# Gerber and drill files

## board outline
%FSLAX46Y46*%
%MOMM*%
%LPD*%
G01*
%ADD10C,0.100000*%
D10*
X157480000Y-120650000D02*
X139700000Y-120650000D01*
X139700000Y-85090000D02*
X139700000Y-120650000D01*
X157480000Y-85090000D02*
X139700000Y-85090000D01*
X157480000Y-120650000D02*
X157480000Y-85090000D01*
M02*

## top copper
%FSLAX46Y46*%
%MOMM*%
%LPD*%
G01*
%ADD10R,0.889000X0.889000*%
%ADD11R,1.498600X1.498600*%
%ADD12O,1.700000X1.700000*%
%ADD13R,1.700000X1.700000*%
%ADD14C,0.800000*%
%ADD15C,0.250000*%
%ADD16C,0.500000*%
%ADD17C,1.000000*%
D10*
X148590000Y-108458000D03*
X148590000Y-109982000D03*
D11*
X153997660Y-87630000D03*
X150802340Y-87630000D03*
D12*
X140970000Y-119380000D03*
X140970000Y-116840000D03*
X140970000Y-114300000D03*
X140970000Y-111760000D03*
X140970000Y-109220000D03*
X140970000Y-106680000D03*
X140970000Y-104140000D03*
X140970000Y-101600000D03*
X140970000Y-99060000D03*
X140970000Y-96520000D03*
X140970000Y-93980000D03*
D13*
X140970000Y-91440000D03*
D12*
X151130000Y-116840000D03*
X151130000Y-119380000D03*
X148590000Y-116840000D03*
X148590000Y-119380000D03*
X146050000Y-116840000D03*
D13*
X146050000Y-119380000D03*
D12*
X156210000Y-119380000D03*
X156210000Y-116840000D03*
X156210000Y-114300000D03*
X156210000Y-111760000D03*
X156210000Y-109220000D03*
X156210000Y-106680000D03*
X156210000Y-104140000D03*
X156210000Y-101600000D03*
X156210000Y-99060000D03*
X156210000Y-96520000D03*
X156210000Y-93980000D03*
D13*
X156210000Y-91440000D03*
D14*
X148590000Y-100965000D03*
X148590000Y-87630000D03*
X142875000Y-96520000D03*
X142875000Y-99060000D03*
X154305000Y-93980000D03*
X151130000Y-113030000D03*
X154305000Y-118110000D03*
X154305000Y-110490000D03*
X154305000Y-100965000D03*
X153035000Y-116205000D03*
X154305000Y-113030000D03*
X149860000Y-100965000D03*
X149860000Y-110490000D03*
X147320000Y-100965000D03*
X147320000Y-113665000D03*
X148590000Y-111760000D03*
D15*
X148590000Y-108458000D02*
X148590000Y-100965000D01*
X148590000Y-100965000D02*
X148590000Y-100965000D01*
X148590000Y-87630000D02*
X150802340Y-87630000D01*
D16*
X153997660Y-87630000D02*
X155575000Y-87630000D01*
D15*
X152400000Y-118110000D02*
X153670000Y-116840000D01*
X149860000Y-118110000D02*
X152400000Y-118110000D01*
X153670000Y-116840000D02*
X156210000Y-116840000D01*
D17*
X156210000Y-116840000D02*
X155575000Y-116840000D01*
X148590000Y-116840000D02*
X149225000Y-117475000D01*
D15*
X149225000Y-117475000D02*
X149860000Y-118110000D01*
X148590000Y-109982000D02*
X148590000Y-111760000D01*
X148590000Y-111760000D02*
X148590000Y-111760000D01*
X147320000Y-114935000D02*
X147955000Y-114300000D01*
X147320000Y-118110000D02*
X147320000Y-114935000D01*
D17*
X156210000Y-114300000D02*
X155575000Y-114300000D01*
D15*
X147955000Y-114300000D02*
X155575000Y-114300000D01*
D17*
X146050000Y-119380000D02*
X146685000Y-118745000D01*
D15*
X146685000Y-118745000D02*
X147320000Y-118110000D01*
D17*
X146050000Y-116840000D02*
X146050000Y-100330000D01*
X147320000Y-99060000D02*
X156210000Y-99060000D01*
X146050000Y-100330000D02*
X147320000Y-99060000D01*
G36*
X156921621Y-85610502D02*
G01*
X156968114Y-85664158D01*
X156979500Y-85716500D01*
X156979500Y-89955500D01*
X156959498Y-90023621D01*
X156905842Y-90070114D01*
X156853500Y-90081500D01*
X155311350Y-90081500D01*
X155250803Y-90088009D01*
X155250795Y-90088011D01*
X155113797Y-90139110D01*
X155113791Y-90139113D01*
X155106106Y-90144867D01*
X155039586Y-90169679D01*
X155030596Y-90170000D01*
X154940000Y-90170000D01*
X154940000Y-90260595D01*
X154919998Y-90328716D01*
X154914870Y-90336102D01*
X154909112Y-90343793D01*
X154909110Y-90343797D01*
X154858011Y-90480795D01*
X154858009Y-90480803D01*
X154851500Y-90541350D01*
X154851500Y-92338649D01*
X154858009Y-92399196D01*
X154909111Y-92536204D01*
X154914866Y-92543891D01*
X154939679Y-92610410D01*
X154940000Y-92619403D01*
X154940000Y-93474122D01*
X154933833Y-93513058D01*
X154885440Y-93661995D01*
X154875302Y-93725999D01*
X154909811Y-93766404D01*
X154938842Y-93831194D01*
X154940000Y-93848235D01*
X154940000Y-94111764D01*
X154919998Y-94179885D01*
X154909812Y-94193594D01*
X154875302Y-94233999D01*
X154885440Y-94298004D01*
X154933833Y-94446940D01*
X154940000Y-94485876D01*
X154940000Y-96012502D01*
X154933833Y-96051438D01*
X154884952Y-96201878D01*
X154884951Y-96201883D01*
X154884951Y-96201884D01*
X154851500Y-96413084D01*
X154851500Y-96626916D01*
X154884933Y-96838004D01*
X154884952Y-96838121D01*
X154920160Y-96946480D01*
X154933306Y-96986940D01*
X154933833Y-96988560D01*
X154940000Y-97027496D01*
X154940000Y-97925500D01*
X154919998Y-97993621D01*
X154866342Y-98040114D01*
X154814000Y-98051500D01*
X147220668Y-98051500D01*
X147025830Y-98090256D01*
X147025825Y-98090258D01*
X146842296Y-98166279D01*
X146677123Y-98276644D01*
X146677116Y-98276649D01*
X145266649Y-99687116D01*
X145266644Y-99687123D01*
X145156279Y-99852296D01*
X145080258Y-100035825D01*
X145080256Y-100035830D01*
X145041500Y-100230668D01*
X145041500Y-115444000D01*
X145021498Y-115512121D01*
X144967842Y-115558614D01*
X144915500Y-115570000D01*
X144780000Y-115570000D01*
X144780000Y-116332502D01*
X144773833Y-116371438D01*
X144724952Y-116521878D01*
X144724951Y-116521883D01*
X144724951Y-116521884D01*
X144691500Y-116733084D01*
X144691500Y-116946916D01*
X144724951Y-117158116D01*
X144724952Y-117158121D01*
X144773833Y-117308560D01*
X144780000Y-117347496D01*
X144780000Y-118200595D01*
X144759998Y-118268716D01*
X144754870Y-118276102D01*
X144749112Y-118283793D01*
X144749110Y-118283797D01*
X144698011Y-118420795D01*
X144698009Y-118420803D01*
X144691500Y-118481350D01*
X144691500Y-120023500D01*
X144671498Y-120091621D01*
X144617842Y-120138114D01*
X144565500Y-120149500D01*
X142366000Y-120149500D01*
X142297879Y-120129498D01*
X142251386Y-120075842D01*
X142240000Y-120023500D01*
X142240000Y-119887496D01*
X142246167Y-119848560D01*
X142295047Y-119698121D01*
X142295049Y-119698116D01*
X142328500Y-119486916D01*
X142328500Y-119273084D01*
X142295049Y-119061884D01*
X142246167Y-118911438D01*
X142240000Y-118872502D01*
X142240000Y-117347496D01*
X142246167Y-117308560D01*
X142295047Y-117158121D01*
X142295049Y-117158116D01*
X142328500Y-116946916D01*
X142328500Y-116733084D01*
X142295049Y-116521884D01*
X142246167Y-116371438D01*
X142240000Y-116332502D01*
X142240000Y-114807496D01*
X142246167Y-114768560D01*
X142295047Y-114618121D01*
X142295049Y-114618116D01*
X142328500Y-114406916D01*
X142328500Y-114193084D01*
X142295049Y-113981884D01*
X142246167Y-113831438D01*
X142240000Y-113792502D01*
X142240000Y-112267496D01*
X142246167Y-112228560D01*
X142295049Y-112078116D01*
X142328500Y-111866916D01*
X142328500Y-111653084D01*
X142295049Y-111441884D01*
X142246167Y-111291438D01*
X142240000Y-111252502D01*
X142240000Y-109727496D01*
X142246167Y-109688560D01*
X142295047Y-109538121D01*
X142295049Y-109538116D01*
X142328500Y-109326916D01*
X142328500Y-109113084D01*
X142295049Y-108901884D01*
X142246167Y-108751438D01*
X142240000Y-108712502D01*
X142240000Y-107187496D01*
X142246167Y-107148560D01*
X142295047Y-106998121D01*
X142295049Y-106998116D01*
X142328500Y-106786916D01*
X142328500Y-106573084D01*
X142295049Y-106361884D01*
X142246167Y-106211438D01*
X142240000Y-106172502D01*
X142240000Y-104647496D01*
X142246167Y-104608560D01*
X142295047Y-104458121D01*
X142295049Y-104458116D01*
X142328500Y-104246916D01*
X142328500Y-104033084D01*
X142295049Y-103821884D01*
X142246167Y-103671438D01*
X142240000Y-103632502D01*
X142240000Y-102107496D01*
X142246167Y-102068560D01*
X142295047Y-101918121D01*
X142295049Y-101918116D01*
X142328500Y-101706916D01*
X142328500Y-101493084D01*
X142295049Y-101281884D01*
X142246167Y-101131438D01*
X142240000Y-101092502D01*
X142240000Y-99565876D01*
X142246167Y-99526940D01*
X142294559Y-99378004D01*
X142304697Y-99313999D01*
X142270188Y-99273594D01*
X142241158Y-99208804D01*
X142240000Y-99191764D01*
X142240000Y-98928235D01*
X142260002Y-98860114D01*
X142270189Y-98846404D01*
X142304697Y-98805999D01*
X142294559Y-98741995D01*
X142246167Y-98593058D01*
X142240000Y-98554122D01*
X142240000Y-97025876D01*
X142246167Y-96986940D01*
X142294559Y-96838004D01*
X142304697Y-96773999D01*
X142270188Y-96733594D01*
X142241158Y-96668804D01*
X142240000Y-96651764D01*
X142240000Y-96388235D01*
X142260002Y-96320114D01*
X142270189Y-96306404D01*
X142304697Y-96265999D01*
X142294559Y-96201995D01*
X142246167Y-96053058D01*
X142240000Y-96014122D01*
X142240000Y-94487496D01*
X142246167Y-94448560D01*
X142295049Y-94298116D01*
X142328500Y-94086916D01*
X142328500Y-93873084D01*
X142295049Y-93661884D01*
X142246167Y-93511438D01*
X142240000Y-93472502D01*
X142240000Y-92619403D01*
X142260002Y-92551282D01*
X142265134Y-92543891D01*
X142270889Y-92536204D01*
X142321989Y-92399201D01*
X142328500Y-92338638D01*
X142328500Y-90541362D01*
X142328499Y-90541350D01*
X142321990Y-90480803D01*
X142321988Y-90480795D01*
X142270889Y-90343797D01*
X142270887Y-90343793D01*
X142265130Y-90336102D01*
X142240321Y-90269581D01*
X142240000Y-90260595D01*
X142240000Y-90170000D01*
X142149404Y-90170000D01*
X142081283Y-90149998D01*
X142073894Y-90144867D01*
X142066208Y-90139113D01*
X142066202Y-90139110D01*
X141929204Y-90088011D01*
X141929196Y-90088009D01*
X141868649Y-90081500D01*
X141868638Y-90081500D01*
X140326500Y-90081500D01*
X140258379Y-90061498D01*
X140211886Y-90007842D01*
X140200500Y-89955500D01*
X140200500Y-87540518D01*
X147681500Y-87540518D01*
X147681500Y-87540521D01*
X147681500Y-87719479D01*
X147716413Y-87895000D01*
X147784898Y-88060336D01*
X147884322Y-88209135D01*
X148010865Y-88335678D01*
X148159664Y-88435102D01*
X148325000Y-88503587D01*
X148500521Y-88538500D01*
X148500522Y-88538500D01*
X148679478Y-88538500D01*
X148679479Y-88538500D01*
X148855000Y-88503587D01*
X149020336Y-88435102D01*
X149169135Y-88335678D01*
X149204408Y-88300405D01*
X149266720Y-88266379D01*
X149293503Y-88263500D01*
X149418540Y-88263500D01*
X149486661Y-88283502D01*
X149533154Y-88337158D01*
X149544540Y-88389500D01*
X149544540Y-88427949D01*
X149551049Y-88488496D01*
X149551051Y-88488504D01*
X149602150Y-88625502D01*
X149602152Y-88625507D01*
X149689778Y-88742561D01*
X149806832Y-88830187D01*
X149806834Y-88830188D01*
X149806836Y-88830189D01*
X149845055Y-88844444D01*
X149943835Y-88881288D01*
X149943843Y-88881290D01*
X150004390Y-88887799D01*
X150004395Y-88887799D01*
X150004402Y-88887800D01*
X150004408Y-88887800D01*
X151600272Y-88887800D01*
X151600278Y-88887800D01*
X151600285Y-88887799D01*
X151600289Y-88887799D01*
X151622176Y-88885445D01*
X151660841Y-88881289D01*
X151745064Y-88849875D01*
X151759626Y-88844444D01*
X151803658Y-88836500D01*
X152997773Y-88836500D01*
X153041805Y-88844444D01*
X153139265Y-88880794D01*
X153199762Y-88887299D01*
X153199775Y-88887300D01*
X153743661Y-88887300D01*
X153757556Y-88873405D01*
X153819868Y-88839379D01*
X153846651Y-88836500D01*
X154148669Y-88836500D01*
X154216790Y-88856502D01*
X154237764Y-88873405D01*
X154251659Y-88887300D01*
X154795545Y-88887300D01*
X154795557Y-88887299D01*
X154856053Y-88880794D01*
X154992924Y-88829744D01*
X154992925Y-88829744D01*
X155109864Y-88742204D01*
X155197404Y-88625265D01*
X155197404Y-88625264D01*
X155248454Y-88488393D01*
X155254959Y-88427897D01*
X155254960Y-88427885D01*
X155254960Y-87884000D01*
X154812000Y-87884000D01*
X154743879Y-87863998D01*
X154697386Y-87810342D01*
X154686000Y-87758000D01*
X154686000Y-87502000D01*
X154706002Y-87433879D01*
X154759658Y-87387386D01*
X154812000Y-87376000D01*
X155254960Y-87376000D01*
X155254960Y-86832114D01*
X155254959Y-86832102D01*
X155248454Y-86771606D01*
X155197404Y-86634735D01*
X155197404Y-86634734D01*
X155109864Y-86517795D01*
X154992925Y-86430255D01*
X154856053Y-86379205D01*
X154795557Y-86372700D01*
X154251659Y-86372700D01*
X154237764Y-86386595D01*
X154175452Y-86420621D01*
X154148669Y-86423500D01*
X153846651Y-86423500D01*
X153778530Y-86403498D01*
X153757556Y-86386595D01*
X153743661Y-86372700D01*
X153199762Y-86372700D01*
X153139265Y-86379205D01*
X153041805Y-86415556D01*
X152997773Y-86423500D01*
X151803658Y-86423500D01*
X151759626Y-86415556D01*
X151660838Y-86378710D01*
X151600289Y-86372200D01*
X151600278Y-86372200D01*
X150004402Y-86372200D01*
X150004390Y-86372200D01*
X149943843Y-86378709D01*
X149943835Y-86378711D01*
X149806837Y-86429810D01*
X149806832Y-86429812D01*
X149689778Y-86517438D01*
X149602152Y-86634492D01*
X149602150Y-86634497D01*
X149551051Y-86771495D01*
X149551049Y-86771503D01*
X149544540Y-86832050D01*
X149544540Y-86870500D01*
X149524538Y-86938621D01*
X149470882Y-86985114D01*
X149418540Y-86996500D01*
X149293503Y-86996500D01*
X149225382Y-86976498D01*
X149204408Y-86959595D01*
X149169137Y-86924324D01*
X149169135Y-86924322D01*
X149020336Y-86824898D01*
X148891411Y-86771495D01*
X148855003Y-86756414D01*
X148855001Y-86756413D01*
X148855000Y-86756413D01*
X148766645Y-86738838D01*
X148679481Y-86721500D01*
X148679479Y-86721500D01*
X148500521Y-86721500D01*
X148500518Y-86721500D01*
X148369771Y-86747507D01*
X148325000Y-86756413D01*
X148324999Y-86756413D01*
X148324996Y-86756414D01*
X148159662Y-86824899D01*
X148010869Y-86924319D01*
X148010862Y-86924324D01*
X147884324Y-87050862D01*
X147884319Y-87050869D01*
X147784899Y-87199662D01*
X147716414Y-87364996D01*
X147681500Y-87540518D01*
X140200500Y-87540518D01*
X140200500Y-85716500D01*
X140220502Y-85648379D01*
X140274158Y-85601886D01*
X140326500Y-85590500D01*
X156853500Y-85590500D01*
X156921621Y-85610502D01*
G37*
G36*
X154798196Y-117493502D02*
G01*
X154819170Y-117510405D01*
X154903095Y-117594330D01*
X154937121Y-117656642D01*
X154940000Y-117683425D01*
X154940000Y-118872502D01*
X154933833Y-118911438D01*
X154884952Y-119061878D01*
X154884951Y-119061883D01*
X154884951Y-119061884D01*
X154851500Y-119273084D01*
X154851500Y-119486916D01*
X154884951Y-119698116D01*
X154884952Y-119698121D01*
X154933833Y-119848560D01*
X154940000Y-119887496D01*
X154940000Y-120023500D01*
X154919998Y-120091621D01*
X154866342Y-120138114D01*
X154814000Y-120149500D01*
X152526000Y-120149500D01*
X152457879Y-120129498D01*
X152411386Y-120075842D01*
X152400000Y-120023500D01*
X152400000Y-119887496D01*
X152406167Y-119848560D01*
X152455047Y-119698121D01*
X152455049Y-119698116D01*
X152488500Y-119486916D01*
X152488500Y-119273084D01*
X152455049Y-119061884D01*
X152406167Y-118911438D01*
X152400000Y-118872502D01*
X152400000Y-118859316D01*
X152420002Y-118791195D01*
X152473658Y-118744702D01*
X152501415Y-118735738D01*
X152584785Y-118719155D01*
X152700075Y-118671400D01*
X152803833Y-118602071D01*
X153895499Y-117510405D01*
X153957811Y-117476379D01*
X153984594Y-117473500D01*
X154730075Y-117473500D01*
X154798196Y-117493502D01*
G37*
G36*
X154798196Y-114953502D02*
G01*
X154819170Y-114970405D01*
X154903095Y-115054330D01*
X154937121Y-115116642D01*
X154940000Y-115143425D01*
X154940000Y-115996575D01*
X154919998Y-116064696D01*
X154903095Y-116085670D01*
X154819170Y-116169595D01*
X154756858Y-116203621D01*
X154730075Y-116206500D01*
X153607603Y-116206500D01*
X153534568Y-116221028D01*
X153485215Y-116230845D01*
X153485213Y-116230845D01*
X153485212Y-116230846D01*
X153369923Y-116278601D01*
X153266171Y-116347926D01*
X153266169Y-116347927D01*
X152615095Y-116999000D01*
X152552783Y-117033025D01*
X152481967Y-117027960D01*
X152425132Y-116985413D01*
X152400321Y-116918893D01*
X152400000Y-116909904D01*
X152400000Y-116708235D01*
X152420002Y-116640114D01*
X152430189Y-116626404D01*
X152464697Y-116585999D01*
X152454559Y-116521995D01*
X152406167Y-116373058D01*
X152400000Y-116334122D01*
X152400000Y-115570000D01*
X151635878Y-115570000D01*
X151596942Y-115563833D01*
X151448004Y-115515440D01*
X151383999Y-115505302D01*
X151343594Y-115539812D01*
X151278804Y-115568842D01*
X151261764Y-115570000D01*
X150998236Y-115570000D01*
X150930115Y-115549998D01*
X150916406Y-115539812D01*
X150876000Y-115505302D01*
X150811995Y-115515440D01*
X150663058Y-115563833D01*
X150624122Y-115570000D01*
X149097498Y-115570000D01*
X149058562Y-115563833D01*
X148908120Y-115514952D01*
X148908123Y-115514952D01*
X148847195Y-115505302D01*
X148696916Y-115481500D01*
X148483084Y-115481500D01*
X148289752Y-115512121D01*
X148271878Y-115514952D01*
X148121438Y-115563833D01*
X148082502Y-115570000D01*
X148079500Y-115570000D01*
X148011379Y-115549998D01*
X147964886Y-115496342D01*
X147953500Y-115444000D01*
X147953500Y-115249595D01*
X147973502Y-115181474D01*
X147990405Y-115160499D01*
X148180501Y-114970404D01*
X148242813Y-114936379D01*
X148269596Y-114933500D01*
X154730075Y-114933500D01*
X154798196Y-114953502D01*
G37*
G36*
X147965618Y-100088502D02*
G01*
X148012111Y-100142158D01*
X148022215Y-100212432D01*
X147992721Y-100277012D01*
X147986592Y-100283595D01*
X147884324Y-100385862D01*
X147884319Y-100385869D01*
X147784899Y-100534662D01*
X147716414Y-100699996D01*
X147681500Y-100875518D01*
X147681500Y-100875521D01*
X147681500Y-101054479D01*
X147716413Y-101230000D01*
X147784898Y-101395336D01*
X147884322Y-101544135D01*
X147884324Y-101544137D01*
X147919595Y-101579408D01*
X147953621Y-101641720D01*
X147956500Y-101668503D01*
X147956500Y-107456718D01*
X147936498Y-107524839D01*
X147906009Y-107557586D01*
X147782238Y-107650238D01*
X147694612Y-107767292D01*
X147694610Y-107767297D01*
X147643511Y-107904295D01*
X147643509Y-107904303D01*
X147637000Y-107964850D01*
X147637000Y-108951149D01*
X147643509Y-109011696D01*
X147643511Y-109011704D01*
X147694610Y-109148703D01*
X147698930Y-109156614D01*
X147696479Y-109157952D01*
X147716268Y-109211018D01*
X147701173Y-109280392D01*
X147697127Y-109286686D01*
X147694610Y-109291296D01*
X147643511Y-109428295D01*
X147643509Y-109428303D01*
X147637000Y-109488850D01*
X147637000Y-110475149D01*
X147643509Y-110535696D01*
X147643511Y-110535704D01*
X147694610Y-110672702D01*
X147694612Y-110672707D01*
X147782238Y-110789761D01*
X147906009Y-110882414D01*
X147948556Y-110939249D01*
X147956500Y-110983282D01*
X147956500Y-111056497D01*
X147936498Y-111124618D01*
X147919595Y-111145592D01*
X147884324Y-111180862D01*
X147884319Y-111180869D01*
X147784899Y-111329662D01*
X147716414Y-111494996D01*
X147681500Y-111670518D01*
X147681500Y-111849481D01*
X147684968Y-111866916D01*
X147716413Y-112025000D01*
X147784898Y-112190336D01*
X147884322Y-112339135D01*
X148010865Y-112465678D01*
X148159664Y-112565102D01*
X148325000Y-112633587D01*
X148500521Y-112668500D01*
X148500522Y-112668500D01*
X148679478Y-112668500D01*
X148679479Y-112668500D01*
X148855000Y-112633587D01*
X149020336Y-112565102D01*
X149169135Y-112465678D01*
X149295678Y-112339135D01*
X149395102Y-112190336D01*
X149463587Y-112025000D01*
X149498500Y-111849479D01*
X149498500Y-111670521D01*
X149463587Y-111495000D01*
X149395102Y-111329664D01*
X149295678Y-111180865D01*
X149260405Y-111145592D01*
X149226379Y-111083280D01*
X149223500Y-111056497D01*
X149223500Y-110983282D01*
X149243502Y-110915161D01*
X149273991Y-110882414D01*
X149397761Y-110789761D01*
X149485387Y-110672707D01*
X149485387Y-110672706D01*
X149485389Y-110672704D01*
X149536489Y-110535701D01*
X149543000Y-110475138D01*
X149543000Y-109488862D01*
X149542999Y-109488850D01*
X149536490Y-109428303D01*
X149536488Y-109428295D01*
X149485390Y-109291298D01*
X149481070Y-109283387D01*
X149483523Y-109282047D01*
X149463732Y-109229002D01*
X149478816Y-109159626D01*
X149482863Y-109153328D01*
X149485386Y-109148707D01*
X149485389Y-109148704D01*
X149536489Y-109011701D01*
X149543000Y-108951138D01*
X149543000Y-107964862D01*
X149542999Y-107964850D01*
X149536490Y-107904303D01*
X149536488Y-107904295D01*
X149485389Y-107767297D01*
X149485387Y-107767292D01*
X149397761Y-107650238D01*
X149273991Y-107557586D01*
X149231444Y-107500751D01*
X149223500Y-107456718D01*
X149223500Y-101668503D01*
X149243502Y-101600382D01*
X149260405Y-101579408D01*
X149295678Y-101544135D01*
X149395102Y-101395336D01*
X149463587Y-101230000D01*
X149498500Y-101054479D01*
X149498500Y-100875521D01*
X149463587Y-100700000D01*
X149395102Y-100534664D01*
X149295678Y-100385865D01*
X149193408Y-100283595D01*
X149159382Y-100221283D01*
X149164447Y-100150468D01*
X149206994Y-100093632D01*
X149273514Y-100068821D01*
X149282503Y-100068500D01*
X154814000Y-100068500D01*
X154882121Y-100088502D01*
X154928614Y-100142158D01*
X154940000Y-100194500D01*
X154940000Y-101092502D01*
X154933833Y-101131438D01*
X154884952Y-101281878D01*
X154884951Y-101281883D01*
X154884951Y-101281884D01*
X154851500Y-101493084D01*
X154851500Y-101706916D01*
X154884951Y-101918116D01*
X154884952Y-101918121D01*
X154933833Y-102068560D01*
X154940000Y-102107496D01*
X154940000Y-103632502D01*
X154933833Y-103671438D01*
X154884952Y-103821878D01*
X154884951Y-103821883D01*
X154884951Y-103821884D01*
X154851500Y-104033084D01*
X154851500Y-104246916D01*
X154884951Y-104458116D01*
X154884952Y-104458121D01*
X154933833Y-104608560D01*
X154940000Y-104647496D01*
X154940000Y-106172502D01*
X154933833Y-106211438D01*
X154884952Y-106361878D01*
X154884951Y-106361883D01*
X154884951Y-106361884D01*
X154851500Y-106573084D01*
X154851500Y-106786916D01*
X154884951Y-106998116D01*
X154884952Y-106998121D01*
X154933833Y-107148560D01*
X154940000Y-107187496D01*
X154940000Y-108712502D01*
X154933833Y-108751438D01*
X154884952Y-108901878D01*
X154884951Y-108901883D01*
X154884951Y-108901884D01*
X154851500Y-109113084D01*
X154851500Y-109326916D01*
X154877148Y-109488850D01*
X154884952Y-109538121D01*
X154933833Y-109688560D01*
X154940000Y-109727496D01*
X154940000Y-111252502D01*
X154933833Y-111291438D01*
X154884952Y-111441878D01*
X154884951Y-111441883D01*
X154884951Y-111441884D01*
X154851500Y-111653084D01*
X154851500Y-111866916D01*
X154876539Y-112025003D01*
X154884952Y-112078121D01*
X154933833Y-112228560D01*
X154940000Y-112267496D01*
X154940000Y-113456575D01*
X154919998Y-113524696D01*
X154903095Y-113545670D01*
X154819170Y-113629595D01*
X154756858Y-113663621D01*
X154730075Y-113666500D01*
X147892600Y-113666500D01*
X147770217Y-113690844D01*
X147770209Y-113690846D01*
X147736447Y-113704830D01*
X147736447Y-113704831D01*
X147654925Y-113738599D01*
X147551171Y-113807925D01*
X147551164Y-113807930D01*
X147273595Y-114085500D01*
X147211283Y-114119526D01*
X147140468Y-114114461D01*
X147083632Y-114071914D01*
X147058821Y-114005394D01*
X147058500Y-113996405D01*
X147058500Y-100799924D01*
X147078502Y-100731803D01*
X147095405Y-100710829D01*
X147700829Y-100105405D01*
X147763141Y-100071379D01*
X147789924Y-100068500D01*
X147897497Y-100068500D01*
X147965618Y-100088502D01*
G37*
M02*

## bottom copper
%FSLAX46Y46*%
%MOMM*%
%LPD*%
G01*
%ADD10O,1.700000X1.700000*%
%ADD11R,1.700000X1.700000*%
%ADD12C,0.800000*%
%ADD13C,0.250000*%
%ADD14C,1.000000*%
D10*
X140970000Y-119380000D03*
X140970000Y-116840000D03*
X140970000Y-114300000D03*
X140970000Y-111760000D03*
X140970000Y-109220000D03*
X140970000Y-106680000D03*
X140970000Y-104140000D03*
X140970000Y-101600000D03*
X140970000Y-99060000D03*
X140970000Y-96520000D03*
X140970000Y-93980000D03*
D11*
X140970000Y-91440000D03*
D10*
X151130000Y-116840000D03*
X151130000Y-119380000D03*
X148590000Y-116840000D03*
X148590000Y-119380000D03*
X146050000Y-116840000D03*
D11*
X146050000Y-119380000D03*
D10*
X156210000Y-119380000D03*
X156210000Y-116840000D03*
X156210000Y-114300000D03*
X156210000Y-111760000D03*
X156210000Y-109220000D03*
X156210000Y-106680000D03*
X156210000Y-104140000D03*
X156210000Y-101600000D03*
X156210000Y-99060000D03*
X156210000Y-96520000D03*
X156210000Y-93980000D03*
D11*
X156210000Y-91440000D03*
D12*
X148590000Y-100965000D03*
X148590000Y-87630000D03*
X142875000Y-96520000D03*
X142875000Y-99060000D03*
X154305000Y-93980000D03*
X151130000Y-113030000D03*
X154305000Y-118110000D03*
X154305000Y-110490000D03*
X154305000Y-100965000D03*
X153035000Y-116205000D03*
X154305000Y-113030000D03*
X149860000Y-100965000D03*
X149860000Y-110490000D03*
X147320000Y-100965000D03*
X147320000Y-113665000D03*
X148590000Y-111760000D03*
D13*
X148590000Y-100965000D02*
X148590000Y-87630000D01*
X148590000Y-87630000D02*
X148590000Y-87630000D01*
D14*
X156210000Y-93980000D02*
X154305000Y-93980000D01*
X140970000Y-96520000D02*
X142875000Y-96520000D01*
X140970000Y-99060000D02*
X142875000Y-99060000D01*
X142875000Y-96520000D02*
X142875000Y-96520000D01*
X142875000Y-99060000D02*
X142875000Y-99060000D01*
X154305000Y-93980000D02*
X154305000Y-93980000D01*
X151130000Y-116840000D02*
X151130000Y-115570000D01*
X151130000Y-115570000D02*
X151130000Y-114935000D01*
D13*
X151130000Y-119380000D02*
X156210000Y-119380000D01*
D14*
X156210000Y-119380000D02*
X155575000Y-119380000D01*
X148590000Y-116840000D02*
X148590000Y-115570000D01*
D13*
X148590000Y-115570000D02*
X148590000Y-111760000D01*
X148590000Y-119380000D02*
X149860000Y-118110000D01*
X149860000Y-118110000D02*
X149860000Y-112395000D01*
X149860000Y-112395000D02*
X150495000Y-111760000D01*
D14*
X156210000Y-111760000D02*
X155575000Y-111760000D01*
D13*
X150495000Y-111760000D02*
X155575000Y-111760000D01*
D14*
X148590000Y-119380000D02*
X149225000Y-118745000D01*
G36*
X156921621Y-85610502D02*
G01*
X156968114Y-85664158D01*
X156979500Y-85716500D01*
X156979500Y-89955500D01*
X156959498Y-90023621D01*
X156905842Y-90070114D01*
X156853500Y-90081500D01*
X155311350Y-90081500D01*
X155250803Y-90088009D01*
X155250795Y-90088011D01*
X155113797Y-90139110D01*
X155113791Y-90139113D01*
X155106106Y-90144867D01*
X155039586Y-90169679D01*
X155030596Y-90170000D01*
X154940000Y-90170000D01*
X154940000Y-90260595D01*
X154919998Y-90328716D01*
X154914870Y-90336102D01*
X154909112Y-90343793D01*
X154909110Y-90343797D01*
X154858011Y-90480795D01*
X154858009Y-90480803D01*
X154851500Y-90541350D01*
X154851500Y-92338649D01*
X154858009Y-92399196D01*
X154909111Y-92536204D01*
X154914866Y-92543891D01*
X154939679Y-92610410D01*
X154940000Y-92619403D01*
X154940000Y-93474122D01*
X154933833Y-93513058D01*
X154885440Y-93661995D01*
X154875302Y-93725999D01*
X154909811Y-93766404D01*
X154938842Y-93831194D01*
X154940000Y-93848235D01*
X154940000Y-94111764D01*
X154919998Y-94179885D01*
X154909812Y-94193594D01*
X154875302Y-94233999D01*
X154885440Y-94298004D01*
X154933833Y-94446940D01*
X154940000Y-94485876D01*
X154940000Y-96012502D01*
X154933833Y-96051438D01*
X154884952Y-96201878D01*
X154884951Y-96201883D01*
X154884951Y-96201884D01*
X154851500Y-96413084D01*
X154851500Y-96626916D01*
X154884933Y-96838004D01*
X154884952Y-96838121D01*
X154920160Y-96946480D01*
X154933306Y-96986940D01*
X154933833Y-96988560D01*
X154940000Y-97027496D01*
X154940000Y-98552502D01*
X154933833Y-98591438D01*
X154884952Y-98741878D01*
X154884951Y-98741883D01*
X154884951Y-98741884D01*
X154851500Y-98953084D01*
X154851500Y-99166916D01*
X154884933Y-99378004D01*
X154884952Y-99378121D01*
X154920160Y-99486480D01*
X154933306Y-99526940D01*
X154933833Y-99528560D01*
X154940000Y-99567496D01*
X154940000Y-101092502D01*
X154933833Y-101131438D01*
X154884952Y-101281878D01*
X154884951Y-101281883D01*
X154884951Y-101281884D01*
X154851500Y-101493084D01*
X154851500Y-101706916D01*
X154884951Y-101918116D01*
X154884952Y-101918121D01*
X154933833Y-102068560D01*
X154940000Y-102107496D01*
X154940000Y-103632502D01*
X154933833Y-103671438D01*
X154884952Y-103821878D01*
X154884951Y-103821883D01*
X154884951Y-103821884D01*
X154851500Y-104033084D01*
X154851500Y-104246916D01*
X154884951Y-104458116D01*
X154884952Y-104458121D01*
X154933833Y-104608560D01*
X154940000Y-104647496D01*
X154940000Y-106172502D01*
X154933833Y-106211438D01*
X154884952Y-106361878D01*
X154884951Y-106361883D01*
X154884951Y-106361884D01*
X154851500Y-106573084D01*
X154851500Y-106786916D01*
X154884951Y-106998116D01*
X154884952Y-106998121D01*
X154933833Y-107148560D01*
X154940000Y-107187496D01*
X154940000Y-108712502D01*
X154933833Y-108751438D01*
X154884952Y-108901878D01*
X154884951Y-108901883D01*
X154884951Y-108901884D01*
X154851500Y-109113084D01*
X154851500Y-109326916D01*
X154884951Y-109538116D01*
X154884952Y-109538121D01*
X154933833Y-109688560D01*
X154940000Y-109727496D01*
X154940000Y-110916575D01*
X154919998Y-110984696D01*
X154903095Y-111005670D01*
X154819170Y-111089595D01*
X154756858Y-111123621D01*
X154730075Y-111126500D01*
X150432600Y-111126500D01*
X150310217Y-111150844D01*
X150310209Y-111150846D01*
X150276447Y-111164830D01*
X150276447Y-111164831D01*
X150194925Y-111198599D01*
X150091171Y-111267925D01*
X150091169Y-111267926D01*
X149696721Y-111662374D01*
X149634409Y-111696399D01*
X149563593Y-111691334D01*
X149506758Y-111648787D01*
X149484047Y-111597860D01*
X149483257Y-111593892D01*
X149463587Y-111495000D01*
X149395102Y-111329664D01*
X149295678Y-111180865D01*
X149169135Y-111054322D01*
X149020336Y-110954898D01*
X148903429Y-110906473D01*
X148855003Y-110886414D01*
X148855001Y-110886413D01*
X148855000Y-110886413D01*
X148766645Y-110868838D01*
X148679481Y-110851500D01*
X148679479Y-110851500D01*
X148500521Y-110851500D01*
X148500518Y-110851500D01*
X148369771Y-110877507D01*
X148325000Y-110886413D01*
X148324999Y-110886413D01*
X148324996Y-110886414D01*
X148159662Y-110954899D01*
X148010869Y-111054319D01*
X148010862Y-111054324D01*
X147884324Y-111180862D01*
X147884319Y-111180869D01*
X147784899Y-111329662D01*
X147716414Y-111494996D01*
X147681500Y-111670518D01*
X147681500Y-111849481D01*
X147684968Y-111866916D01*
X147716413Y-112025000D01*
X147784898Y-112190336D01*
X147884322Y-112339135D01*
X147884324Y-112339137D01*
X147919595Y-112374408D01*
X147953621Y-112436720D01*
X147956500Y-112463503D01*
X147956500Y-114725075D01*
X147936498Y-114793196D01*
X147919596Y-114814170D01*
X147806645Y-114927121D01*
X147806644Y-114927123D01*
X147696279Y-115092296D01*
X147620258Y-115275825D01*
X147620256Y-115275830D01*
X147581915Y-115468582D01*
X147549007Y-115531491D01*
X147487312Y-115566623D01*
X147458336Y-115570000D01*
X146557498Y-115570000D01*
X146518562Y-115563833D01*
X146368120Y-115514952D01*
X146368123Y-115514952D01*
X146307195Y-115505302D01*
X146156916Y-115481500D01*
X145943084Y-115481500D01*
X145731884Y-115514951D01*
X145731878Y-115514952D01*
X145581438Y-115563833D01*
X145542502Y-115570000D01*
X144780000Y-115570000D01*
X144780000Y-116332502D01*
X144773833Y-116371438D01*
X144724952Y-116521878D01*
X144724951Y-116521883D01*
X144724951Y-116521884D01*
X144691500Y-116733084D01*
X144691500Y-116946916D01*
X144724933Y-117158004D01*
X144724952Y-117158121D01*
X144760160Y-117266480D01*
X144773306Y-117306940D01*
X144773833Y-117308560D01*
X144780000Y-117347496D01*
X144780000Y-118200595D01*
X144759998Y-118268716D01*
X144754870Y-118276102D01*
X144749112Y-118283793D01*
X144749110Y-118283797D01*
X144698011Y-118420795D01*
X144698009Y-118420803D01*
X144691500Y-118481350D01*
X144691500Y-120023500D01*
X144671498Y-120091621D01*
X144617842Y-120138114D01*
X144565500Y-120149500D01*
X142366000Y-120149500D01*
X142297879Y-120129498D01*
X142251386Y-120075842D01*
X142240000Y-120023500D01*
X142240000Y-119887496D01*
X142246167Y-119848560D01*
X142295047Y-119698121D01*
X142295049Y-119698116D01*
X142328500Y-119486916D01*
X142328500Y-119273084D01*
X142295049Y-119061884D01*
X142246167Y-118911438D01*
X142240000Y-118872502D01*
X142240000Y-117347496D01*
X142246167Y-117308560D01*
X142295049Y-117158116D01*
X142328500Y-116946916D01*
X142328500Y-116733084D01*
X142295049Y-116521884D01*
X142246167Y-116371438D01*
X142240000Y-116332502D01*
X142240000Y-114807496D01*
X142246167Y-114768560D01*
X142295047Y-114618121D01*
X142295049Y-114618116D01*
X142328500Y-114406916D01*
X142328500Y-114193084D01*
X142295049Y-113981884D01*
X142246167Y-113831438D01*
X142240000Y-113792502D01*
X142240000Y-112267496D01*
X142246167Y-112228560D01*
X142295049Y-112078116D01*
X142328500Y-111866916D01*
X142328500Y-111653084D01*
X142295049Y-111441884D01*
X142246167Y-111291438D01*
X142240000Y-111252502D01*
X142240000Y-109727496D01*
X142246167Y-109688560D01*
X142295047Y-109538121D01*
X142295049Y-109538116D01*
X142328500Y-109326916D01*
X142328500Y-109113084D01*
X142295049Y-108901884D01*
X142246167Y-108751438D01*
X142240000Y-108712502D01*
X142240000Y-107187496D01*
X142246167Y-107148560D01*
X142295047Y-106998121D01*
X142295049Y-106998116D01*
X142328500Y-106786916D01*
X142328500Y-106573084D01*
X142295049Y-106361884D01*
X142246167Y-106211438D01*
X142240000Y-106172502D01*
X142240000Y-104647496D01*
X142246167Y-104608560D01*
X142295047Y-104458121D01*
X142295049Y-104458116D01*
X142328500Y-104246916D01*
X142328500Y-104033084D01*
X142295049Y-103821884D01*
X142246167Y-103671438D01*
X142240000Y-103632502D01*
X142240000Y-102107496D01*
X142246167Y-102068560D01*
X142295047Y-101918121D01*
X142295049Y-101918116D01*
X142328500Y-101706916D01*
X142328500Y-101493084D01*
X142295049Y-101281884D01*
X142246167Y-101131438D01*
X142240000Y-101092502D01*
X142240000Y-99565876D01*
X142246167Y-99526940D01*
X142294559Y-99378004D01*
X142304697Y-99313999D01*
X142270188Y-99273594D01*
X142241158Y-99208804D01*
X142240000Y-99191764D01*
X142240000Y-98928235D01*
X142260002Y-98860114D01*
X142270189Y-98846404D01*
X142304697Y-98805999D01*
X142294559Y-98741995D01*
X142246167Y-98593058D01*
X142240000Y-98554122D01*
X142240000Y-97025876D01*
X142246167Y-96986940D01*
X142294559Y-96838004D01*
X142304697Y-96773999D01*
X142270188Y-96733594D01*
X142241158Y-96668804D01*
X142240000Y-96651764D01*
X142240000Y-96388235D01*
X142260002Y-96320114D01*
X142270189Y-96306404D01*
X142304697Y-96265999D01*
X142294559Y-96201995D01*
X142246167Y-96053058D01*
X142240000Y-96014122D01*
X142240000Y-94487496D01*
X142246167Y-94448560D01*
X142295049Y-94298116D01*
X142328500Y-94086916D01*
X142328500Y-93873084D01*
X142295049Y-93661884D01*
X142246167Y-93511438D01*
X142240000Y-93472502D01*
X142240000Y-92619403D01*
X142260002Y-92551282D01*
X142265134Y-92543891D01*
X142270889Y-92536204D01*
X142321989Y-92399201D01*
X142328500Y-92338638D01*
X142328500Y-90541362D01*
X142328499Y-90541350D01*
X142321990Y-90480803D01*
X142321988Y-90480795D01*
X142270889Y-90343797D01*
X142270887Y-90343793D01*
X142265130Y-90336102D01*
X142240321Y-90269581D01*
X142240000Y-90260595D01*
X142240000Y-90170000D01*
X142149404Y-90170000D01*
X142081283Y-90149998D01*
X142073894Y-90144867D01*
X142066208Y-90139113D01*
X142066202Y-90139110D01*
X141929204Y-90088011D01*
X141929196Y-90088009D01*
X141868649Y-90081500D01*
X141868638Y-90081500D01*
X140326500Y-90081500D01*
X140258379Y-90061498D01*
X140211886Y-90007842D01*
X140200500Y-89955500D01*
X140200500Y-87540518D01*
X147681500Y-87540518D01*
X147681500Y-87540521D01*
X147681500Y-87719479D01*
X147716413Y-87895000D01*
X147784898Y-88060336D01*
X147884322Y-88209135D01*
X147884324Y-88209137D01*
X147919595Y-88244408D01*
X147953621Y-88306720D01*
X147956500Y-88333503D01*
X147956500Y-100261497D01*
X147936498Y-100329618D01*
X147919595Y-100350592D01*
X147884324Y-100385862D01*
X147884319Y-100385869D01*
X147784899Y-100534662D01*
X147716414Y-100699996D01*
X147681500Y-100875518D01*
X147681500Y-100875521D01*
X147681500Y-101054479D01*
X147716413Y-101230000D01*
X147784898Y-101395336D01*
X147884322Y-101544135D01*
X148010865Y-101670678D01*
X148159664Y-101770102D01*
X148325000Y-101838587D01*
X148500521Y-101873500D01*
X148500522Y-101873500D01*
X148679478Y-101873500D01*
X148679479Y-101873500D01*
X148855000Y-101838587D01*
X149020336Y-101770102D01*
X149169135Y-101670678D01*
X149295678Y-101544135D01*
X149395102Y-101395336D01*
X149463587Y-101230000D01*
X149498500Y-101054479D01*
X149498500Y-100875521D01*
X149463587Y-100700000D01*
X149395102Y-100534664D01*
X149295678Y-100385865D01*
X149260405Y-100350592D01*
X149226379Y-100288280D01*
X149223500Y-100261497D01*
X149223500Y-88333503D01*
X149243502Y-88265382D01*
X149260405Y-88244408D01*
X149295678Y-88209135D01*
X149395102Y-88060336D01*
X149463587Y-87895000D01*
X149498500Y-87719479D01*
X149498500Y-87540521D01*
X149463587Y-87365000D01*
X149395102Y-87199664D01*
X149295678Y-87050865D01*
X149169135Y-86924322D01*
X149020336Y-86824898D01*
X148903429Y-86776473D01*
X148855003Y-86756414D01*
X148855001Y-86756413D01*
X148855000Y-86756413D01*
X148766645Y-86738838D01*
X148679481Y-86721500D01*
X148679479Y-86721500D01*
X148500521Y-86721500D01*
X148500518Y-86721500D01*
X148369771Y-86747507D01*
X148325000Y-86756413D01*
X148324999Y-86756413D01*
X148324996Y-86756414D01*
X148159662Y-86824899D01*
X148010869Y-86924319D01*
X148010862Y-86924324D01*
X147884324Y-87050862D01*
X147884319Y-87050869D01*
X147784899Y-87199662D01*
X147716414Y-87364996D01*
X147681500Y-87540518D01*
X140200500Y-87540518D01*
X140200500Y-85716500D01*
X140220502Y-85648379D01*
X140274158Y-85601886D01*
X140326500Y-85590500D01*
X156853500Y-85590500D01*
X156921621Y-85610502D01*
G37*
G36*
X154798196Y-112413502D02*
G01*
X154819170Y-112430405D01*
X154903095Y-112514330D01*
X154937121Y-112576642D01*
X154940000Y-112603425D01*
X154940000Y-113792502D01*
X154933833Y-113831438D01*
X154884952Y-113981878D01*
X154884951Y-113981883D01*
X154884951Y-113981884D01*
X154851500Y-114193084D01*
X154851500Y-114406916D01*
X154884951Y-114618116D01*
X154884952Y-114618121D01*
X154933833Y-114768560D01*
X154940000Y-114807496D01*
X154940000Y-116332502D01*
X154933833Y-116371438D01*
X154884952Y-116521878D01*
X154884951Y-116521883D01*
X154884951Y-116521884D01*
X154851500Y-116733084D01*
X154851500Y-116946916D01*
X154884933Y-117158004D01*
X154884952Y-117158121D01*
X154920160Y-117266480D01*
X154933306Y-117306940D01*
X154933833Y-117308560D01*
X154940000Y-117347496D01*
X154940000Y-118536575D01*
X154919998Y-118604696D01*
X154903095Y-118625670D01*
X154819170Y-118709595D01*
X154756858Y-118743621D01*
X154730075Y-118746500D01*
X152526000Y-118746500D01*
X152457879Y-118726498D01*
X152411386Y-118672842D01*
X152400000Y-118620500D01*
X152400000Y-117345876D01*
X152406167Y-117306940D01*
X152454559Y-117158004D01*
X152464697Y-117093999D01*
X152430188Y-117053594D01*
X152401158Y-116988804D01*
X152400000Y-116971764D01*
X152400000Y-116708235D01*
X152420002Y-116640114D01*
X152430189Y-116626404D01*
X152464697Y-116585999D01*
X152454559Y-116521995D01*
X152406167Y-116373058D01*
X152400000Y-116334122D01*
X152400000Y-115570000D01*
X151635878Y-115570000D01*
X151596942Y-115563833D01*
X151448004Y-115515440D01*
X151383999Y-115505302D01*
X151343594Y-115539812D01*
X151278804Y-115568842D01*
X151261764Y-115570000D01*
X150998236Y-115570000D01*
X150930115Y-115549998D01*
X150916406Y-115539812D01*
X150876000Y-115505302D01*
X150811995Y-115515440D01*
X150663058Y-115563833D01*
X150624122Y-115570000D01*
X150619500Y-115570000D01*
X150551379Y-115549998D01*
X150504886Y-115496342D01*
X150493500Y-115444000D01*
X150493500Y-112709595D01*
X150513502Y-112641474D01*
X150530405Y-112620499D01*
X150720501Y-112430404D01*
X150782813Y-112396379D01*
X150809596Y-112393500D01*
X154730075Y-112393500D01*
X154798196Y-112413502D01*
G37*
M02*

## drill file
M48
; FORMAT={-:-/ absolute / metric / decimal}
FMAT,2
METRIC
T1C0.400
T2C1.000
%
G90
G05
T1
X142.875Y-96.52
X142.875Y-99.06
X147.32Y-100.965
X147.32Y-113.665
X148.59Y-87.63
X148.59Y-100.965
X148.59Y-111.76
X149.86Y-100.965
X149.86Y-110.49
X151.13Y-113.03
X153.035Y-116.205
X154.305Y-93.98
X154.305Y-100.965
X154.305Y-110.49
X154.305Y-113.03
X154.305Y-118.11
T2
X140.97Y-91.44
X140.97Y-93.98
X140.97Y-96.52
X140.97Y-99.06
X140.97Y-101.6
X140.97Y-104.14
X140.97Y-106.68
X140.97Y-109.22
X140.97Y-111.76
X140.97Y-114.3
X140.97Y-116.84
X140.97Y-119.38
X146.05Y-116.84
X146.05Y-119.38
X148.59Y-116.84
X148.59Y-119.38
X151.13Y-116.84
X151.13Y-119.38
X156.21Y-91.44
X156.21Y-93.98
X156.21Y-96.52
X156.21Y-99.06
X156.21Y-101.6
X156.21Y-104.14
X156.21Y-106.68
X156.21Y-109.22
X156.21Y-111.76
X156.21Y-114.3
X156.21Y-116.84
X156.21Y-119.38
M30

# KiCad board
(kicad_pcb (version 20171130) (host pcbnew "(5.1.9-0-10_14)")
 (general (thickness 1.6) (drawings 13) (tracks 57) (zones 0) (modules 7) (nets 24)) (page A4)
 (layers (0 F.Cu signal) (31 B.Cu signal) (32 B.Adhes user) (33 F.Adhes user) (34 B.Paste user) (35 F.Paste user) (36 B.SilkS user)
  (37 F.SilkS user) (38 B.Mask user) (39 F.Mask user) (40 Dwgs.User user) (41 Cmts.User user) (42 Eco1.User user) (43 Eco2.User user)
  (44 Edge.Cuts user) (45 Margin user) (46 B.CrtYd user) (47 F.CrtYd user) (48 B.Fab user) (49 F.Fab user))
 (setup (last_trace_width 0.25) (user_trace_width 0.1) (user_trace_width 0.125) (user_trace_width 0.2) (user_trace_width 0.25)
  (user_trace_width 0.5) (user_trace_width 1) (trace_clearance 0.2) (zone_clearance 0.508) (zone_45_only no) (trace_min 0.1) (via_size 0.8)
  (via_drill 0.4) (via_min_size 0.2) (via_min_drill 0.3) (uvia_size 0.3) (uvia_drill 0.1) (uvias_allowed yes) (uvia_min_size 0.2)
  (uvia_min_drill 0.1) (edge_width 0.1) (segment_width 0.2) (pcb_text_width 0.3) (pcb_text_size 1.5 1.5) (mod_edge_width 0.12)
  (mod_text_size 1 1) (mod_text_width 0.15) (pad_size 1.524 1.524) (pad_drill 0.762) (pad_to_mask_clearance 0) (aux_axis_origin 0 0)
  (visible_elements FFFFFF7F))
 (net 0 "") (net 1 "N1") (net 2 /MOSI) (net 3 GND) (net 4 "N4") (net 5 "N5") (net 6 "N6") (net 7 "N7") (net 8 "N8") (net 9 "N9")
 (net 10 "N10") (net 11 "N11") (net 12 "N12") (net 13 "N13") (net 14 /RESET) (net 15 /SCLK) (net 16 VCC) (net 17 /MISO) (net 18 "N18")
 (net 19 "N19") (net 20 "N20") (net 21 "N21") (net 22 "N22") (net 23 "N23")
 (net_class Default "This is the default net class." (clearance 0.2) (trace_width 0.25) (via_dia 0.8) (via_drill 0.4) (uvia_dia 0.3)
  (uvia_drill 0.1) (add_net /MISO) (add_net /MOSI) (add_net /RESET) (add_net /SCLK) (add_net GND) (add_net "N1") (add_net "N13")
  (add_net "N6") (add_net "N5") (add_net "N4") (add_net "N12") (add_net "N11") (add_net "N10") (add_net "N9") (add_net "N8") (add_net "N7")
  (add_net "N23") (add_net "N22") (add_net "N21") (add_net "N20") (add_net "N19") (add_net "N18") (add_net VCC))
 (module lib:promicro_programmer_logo (layer B.Cu) (at 146.05 93.98 270)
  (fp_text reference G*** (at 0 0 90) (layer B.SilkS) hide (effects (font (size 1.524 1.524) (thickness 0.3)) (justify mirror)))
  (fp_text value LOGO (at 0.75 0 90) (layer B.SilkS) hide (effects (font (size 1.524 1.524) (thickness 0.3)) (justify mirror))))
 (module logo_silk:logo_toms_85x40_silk (layer B.Cu) (at 146.685 106.68 270)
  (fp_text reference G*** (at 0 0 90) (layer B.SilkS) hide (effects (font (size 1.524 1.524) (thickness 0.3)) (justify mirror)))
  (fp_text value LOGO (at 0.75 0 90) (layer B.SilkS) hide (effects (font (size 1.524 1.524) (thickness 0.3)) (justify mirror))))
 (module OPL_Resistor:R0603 (layer F.Cu) (at 148.59 109.22 90)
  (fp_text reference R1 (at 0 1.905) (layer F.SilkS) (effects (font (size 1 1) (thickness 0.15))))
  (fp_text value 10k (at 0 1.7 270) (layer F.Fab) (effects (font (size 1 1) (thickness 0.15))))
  (pad 2 smd rect (at 0.762 0 90) (size 0.889 0.889) (layers F.Cu F.Paste F.Mask) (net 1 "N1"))
  (pad 1 smd rect (at -0.762 0 90) (size 0.889 0.889) (layers F.Cu F.Paste F.Mask) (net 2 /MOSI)))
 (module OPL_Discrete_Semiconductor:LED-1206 (layer F.Cu) (at 152.4 87.63 180)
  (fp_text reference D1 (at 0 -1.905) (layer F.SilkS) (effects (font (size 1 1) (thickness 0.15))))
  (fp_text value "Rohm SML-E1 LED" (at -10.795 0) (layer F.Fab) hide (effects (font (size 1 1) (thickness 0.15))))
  (pad 1 smd rect (at -1.59766 0 180) (size 1.4986 1.4986) (layers F.Cu F.Paste F.Mask) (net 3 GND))
  (pad 2 smd rect (at 1.59766 0 180) (size 1.4986 1.4986) (layers F.Cu F.Paste F.Mask) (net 1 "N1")))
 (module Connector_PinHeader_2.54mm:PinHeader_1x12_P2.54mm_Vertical (layer F.Cu) (at 140.97 91.44)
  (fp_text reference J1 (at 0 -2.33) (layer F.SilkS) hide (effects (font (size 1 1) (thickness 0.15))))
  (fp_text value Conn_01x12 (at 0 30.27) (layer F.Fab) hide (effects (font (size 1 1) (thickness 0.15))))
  (pad 12 thru_hole oval (at 0 27.94) (size 1.7 1.7) (drill 1) (layers *.Cu *.Mask) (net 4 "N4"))
  (pad 11 thru_hole oval (at 0 25.4) (size 1.7 1.7) (drill 1) (layers *.Cu *.Mask) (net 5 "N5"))
  (pad 10 thru_hole oval (at 0 22.86) (size 1.7 1.7) (drill 1) (layers *.Cu *.Mask) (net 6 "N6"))
  (pad 9 thru_hole oval (at 0 20.32) (size 1.7 1.7) (drill 1) (layers *.Cu *.Mask) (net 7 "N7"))
  (pad 8 thru_hole oval (at 0 17.78) (size 1.7 1.7) (drill 1) (layers *.Cu *.Mask) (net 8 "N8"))
  (pad 7 thru_hole oval (at 0 15.24) (size 1.7 1.7) (drill 1) (layers *.Cu *.Mask) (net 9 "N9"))
  (pad 6 thru_hole oval (at 0 12.7) (size 1.7 1.7) (drill 1) (layers *.Cu *.Mask) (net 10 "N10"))
  (pad 5 thru_hole oval (at 0 10.16) (size 1.7 1.7) (drill 1) (layers *.Cu *.Mask) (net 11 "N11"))
  (pad 4 thru_hole oval (at 0 7.62) (size 1.7 1.7) (drill 1) (layers *.Cu *.Mask) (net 3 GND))
  (pad 3 thru_hole oval (at 0 5.08) (size 1.7 1.7) (drill 1) (layers *.Cu *.Mask) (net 3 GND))
  (pad 2 thru_hole oval (at 0 2.54) (size 1.7 1.7) (drill 1) (layers *.Cu *.Mask) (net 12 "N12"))
  (pad 1 thru_hole rect (at 0 0) (size 1.7 1.7) (drill 1) (layers *.Cu *.Mask) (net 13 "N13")))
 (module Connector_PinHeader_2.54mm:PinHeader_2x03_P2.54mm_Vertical (layer F.Cu) (at 146.05 119.38 90)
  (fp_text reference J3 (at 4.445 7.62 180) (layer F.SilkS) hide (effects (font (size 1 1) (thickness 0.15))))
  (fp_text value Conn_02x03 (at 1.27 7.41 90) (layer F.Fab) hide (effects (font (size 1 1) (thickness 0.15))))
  (pad 6 thru_hole oval (at 2.54 5.08 90) (size 1.7 1.7) (drill 1) (layers *.Cu *.Mask) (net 3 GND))
  (pad 5 thru_hole oval (at 0 5.08 90) (size 1.7 1.7) (drill 1) (layers *.Cu *.Mask) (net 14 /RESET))
  (pad 4 thru_hole oval (at 2.54 2.54 90) (size 1.7 1.7) (drill 1) (layers *.Cu *.Mask) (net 2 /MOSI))
  (pad 3 thru_hole oval (at 0 2.54 90) (size 1.7 1.7) (drill 1) (layers *.Cu *.Mask) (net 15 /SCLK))
  (pad 2 thru_hole oval (at 2.54 0 90) (size 1.7 1.7) (drill 1) (layers *.Cu *.Mask) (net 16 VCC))
  (pad 1 thru_hole rect (at 0 0 90) (size 1.7 1.7) (drill 1) (layers *.Cu *.Mask) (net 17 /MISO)))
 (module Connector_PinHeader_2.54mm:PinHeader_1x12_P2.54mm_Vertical (layer F.Cu) (at 156.21 91.44)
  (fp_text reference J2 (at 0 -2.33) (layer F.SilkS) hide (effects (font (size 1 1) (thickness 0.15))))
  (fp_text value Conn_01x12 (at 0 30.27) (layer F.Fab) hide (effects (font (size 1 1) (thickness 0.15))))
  (pad 12 thru_hole oval (at 0 27.94) (size 1.7 1.7) (drill 1) (layers *.Cu *.Mask) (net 14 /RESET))
  (pad 11 thru_hole oval (at 0 25.4) (size 1.7 1.7) (drill 1) (layers *.Cu *.Mask) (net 2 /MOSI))
  (pad 10 thru_hole oval (at 0 22.86) (size 1.7 1.7) (drill 1) (layers *.Cu *.Mask) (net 17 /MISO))
  (pad 9 thru_hole oval (at 0 20.32) (size 1.7 1.7) (drill 1) (layers *.Cu *.Mask) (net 15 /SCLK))
  (pad 8 thru_hole oval (at 0 17.78) (size 1.7 1.7) (drill 1) (layers *.Cu *.Mask) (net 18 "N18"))
  (pad 7 thru_hole oval (at 0 15.24) (size 1.7 1.7) (drill 1) (layers *.Cu *.Mask) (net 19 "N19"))
  (pad 6 thru_hole oval (at 0 12.7) (size 1.7 1.7) (drill 1) (layers *.Cu *.Mask) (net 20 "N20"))
  (pad 5 thru_hole oval (at 0 10.16) (size 1.7 1.7) (drill 1) (layers *.Cu *.Mask) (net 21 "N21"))
  (pad 4 thru_hole oval (at 0 7.62) (size 1.7 1.7) (drill 1) (layers *.Cu *.Mask) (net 16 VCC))
  (pad 3 thru_hole oval (at 0 5.08) (size 1.7 1.7) (drill 1) (layers *.Cu *.Mask) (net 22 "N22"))
  (pad 2 thru_hole oval (at 0 2.54) (size 1.7 1.7) (drill 1) (layers *.Cu *.Mask) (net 3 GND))
  (pad 1 thru_hole rect (at 0 0) (size 1.7 1.7) (drill 1) (layers *.Cu *.Mask) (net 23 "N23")))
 (gr_line (start 157.48 120.65) (end 139.7 120.65) (layer Edge.Cuts) (width 0.1))
 (gr_line (start 139.7 85.09) (end 139.7 120.65) (layer Edge.Cuts) (width 0.1))
 (gr_line (start 157.48 85.09) (end 139.7 85.09) (layer Edge.Cuts) (width 0.1))
 (gr_line (start 157.48 120.65) (end 157.48 85.09) (layer Edge.Cuts) (width 0.1))
 (segment (start 148.59 108.458) (end 148.59 100.965) (width 0.25) (layer F.Cu) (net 1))
 (segment (start 148.59 100.965) (end 148.59 100.965) (width 0.25) (layer F.Cu) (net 1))
 (via (at 148.59 100.965) (size 0.8) (drill 0.4) (layers F.Cu B.Cu) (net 1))
 (segment (start 148.59 100.965) (end 148.59 87.63) (width 0.25) (layer B.Cu) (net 1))
 (segment (start 148.59 87.63) (end 148.59 87.63) (width 0.25) (layer B.Cu) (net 1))
 (via (at 148.59 87.63) (size 0.8) (drill 0.4) (layers F.Cu B.Cu) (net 1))
 (segment (start 148.59 87.63) (end 150.80234 87.63) (width 0.25) (layer F.Cu) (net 1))
 (segment (start 156.21 93.98) (end 154.305 93.98) (width 1) (layer B.Cu) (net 3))
 (segment (start 140.97 96.52) (end 142.875 96.52) (width 1) (layer B.Cu) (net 3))
 (segment (start 140.97 99.06) (end 142.875 99.06) (width 1) (layer B.Cu) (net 3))
 (segment (start 142.875 96.52) (end 142.875 96.52) (width 1) (layer B.Cu) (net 3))
 (via (at 142.875 96.52) (size 0.8) (drill 0.4) (layers F.Cu B.Cu) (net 3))
 (segment (start 142.875 99.06) (end 142.875 99.06) (width 1) (layer B.Cu) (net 3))
 (via (at 142.875 99.06) (size 0.8) (drill 0.4) (layers F.Cu B.Cu) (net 3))
 (segment (start 154.305 93.98) (end 154.305 93.98) (width 1) (layer B.Cu) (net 3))
 (via (at 154.305 93.98) (size 0.8) (drill 0.4) (layers F.Cu B.Cu) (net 3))
 (via (at 151.13 113.03) (size 0.8) (drill 0.4) (layers F.Cu B.Cu) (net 3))
 (via (at 154.305 118.11) (size 0.8) (drill 0.4) (layers F.Cu B.Cu) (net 3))
 (segment (start 151.13 116.84) (end 151.13 115.57) (width 1) (layer B.Cu) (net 3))
 (via (at 154.305 110.49) (size 0.8) (drill 0.4) (layers F.Cu B.Cu) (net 3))
 (via (at 154.305 100.965) (size 0.8) (drill 0.4) (layers F.Cu B.Cu) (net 3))
 (segment (start 151.13 115.57) (end 151.13 114.935) (width 1) (layer B.Cu) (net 3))
 (via (at 153.035 116.205) (size 0.8) (drill 0.4) (layers F.Cu B.Cu) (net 3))
 (via (at 154.305 113.03) (size 0.8) (drill 0.4) (layers F.Cu B.Cu) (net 3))
 (via (at 149.86 100.965) (size 0.8) (drill 0.4) (layers F.Cu B.Cu) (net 3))
 (via (at 149.86 110.49) (size 0.8) (drill 0.4) (layers F.Cu B.Cu) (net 3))
 (via (at 147.32 100.965) (size 0.8) (drill 0.4) (layers F.Cu B.Cu) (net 3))
 (via (at 147.32 113.665) (size 0.8) (drill 0.4) (layers F.Cu B.Cu) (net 3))
 (segment (start 153.99766 87.63) (end 155.575 87.63) (width 0.5) (layer F.Cu) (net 3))
 (segment (start 151.13 119.38) (end 156.21 119.38) (width 0.25) (layer B.Cu) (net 14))
 (segment (start 156.21 119.38) (end 155.575 119.38) (width 1) (layer B.Cu) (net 14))
 (segment (start 152.4 118.11) (end 153.67 116.84) (width 0.25) (layer F.Cu) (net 2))
 (segment (start 149.86 118.11) (end 152.4 118.11) (width 0.25) (layer F.Cu) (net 2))
 (segment (start 153.67 116.84) (end 156.21 116.84) (width 0.25) (layer F.Cu) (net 2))
 (segment (start 156.21 116.84) (end 155.575 116.84) (width 1) (layer F.Cu) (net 2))
 (segment (start 148.59 116.84) (end 149.225 117.475) (width 1) (layer F.Cu) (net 2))
 (segment (start 149.225 117.475) (end 149.86 118.11) (width 0.25) (layer F.Cu) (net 2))
 (segment (start 148.59 116.84) (end 148.59 115.57) (width 1) (layer B.Cu) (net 2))
 (segment (start 148.59 109.982) (end 148.59 111.76) (width 0.25) (layer F.Cu) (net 2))
 (segment (start 148.59 111.76) (end 148.59 111.76) (width 0.25) (layer F.Cu) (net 2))
 (via (at 148.59 111.76) (size 0.8) (drill 0.4) (layers F.Cu B.Cu) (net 2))
 (segment (start 148.59 115.57) (end 148.59 111.76) (width 0.25) (layer B.Cu) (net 2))
 (segment (start 147.32 114.935) (end 147.955 114.3) (width 0.25) (layer F.Cu) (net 17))
 (segment (start 147.32 118.11) (end 147.32 114.935) (width 0.25) (layer F.Cu) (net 17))
 (segment (start 156.21 114.3) (end 155.575 114.3) (width 1) (layer F.Cu) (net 17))
 (segment (start 147.955 114.3) (end 155.575 114.3) (width 0.25) (layer F.Cu) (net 17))
 (segment (start 146.05 119.38) (end 146.685 118.745) (width 1) (layer F.Cu) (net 17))
 (segment (start 146.685 118.745) (end 147.32 118.11) (width 0.25) (layer F.Cu) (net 17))
 (segment (start 148.59 119.38) (end 149.86 118.11) (width 0.25) (layer B.Cu) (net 15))
 (segment (start 149.86 118.11) (end 149.86 112.395) (width 0.25) (layer B.Cu) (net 15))
 (segment (start 149.86 112.395) (end 150.495 111.76) (width 0.25) (layer B.Cu) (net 15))
 (segment (start 156.21 111.76) (end 155.575 111.76) (width 1) (layer B.Cu) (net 15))
 (segment (start 150.495 111.76) (end 155.575 111.76) (width 0.25) (layer B.Cu) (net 15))
 (segment (start 148.59 119.38) (end 149.225 118.745) (width 1) (layer B.Cu) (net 15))
 (segment (start 146.05 116.84) (end 146.05 100.33) (width 1) (layer F.Cu) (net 16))
 (segment (start 147.32 99.06) (end 156.21 99.06) (width 1) (layer F.Cu) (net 16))
 (segment (start 146.05 100.33) (end 147.32 99.06) (width 1) (layer F.Cu) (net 16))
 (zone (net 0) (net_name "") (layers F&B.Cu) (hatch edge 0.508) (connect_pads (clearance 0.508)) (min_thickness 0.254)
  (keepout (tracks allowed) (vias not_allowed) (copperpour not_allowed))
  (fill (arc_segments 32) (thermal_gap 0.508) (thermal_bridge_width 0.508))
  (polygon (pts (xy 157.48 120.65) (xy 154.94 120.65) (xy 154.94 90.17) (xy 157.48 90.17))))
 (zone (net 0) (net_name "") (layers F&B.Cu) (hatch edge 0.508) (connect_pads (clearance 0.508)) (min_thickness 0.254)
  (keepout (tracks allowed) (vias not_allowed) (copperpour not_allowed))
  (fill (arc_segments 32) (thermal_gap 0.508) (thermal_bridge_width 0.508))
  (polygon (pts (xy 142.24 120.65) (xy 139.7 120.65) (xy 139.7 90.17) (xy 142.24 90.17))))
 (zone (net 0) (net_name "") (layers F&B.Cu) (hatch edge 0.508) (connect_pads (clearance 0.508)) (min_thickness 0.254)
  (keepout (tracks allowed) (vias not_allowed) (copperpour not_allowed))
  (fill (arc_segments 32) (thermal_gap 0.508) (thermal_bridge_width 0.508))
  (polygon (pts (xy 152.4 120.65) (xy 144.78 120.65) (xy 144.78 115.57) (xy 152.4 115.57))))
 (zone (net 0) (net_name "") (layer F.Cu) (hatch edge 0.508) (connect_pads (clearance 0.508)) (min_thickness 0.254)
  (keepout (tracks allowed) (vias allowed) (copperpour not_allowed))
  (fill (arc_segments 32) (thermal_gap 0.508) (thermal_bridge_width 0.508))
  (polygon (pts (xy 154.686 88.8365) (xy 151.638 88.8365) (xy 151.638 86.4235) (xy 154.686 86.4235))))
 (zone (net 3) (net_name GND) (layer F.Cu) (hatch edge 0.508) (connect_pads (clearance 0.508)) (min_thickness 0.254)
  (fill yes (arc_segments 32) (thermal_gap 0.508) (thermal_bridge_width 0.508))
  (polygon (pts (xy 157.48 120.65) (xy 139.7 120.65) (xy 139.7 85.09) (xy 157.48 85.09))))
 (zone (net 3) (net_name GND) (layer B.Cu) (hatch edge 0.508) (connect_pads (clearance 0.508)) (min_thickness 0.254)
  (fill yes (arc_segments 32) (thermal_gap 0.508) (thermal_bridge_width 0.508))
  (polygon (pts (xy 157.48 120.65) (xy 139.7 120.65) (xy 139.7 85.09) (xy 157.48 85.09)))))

